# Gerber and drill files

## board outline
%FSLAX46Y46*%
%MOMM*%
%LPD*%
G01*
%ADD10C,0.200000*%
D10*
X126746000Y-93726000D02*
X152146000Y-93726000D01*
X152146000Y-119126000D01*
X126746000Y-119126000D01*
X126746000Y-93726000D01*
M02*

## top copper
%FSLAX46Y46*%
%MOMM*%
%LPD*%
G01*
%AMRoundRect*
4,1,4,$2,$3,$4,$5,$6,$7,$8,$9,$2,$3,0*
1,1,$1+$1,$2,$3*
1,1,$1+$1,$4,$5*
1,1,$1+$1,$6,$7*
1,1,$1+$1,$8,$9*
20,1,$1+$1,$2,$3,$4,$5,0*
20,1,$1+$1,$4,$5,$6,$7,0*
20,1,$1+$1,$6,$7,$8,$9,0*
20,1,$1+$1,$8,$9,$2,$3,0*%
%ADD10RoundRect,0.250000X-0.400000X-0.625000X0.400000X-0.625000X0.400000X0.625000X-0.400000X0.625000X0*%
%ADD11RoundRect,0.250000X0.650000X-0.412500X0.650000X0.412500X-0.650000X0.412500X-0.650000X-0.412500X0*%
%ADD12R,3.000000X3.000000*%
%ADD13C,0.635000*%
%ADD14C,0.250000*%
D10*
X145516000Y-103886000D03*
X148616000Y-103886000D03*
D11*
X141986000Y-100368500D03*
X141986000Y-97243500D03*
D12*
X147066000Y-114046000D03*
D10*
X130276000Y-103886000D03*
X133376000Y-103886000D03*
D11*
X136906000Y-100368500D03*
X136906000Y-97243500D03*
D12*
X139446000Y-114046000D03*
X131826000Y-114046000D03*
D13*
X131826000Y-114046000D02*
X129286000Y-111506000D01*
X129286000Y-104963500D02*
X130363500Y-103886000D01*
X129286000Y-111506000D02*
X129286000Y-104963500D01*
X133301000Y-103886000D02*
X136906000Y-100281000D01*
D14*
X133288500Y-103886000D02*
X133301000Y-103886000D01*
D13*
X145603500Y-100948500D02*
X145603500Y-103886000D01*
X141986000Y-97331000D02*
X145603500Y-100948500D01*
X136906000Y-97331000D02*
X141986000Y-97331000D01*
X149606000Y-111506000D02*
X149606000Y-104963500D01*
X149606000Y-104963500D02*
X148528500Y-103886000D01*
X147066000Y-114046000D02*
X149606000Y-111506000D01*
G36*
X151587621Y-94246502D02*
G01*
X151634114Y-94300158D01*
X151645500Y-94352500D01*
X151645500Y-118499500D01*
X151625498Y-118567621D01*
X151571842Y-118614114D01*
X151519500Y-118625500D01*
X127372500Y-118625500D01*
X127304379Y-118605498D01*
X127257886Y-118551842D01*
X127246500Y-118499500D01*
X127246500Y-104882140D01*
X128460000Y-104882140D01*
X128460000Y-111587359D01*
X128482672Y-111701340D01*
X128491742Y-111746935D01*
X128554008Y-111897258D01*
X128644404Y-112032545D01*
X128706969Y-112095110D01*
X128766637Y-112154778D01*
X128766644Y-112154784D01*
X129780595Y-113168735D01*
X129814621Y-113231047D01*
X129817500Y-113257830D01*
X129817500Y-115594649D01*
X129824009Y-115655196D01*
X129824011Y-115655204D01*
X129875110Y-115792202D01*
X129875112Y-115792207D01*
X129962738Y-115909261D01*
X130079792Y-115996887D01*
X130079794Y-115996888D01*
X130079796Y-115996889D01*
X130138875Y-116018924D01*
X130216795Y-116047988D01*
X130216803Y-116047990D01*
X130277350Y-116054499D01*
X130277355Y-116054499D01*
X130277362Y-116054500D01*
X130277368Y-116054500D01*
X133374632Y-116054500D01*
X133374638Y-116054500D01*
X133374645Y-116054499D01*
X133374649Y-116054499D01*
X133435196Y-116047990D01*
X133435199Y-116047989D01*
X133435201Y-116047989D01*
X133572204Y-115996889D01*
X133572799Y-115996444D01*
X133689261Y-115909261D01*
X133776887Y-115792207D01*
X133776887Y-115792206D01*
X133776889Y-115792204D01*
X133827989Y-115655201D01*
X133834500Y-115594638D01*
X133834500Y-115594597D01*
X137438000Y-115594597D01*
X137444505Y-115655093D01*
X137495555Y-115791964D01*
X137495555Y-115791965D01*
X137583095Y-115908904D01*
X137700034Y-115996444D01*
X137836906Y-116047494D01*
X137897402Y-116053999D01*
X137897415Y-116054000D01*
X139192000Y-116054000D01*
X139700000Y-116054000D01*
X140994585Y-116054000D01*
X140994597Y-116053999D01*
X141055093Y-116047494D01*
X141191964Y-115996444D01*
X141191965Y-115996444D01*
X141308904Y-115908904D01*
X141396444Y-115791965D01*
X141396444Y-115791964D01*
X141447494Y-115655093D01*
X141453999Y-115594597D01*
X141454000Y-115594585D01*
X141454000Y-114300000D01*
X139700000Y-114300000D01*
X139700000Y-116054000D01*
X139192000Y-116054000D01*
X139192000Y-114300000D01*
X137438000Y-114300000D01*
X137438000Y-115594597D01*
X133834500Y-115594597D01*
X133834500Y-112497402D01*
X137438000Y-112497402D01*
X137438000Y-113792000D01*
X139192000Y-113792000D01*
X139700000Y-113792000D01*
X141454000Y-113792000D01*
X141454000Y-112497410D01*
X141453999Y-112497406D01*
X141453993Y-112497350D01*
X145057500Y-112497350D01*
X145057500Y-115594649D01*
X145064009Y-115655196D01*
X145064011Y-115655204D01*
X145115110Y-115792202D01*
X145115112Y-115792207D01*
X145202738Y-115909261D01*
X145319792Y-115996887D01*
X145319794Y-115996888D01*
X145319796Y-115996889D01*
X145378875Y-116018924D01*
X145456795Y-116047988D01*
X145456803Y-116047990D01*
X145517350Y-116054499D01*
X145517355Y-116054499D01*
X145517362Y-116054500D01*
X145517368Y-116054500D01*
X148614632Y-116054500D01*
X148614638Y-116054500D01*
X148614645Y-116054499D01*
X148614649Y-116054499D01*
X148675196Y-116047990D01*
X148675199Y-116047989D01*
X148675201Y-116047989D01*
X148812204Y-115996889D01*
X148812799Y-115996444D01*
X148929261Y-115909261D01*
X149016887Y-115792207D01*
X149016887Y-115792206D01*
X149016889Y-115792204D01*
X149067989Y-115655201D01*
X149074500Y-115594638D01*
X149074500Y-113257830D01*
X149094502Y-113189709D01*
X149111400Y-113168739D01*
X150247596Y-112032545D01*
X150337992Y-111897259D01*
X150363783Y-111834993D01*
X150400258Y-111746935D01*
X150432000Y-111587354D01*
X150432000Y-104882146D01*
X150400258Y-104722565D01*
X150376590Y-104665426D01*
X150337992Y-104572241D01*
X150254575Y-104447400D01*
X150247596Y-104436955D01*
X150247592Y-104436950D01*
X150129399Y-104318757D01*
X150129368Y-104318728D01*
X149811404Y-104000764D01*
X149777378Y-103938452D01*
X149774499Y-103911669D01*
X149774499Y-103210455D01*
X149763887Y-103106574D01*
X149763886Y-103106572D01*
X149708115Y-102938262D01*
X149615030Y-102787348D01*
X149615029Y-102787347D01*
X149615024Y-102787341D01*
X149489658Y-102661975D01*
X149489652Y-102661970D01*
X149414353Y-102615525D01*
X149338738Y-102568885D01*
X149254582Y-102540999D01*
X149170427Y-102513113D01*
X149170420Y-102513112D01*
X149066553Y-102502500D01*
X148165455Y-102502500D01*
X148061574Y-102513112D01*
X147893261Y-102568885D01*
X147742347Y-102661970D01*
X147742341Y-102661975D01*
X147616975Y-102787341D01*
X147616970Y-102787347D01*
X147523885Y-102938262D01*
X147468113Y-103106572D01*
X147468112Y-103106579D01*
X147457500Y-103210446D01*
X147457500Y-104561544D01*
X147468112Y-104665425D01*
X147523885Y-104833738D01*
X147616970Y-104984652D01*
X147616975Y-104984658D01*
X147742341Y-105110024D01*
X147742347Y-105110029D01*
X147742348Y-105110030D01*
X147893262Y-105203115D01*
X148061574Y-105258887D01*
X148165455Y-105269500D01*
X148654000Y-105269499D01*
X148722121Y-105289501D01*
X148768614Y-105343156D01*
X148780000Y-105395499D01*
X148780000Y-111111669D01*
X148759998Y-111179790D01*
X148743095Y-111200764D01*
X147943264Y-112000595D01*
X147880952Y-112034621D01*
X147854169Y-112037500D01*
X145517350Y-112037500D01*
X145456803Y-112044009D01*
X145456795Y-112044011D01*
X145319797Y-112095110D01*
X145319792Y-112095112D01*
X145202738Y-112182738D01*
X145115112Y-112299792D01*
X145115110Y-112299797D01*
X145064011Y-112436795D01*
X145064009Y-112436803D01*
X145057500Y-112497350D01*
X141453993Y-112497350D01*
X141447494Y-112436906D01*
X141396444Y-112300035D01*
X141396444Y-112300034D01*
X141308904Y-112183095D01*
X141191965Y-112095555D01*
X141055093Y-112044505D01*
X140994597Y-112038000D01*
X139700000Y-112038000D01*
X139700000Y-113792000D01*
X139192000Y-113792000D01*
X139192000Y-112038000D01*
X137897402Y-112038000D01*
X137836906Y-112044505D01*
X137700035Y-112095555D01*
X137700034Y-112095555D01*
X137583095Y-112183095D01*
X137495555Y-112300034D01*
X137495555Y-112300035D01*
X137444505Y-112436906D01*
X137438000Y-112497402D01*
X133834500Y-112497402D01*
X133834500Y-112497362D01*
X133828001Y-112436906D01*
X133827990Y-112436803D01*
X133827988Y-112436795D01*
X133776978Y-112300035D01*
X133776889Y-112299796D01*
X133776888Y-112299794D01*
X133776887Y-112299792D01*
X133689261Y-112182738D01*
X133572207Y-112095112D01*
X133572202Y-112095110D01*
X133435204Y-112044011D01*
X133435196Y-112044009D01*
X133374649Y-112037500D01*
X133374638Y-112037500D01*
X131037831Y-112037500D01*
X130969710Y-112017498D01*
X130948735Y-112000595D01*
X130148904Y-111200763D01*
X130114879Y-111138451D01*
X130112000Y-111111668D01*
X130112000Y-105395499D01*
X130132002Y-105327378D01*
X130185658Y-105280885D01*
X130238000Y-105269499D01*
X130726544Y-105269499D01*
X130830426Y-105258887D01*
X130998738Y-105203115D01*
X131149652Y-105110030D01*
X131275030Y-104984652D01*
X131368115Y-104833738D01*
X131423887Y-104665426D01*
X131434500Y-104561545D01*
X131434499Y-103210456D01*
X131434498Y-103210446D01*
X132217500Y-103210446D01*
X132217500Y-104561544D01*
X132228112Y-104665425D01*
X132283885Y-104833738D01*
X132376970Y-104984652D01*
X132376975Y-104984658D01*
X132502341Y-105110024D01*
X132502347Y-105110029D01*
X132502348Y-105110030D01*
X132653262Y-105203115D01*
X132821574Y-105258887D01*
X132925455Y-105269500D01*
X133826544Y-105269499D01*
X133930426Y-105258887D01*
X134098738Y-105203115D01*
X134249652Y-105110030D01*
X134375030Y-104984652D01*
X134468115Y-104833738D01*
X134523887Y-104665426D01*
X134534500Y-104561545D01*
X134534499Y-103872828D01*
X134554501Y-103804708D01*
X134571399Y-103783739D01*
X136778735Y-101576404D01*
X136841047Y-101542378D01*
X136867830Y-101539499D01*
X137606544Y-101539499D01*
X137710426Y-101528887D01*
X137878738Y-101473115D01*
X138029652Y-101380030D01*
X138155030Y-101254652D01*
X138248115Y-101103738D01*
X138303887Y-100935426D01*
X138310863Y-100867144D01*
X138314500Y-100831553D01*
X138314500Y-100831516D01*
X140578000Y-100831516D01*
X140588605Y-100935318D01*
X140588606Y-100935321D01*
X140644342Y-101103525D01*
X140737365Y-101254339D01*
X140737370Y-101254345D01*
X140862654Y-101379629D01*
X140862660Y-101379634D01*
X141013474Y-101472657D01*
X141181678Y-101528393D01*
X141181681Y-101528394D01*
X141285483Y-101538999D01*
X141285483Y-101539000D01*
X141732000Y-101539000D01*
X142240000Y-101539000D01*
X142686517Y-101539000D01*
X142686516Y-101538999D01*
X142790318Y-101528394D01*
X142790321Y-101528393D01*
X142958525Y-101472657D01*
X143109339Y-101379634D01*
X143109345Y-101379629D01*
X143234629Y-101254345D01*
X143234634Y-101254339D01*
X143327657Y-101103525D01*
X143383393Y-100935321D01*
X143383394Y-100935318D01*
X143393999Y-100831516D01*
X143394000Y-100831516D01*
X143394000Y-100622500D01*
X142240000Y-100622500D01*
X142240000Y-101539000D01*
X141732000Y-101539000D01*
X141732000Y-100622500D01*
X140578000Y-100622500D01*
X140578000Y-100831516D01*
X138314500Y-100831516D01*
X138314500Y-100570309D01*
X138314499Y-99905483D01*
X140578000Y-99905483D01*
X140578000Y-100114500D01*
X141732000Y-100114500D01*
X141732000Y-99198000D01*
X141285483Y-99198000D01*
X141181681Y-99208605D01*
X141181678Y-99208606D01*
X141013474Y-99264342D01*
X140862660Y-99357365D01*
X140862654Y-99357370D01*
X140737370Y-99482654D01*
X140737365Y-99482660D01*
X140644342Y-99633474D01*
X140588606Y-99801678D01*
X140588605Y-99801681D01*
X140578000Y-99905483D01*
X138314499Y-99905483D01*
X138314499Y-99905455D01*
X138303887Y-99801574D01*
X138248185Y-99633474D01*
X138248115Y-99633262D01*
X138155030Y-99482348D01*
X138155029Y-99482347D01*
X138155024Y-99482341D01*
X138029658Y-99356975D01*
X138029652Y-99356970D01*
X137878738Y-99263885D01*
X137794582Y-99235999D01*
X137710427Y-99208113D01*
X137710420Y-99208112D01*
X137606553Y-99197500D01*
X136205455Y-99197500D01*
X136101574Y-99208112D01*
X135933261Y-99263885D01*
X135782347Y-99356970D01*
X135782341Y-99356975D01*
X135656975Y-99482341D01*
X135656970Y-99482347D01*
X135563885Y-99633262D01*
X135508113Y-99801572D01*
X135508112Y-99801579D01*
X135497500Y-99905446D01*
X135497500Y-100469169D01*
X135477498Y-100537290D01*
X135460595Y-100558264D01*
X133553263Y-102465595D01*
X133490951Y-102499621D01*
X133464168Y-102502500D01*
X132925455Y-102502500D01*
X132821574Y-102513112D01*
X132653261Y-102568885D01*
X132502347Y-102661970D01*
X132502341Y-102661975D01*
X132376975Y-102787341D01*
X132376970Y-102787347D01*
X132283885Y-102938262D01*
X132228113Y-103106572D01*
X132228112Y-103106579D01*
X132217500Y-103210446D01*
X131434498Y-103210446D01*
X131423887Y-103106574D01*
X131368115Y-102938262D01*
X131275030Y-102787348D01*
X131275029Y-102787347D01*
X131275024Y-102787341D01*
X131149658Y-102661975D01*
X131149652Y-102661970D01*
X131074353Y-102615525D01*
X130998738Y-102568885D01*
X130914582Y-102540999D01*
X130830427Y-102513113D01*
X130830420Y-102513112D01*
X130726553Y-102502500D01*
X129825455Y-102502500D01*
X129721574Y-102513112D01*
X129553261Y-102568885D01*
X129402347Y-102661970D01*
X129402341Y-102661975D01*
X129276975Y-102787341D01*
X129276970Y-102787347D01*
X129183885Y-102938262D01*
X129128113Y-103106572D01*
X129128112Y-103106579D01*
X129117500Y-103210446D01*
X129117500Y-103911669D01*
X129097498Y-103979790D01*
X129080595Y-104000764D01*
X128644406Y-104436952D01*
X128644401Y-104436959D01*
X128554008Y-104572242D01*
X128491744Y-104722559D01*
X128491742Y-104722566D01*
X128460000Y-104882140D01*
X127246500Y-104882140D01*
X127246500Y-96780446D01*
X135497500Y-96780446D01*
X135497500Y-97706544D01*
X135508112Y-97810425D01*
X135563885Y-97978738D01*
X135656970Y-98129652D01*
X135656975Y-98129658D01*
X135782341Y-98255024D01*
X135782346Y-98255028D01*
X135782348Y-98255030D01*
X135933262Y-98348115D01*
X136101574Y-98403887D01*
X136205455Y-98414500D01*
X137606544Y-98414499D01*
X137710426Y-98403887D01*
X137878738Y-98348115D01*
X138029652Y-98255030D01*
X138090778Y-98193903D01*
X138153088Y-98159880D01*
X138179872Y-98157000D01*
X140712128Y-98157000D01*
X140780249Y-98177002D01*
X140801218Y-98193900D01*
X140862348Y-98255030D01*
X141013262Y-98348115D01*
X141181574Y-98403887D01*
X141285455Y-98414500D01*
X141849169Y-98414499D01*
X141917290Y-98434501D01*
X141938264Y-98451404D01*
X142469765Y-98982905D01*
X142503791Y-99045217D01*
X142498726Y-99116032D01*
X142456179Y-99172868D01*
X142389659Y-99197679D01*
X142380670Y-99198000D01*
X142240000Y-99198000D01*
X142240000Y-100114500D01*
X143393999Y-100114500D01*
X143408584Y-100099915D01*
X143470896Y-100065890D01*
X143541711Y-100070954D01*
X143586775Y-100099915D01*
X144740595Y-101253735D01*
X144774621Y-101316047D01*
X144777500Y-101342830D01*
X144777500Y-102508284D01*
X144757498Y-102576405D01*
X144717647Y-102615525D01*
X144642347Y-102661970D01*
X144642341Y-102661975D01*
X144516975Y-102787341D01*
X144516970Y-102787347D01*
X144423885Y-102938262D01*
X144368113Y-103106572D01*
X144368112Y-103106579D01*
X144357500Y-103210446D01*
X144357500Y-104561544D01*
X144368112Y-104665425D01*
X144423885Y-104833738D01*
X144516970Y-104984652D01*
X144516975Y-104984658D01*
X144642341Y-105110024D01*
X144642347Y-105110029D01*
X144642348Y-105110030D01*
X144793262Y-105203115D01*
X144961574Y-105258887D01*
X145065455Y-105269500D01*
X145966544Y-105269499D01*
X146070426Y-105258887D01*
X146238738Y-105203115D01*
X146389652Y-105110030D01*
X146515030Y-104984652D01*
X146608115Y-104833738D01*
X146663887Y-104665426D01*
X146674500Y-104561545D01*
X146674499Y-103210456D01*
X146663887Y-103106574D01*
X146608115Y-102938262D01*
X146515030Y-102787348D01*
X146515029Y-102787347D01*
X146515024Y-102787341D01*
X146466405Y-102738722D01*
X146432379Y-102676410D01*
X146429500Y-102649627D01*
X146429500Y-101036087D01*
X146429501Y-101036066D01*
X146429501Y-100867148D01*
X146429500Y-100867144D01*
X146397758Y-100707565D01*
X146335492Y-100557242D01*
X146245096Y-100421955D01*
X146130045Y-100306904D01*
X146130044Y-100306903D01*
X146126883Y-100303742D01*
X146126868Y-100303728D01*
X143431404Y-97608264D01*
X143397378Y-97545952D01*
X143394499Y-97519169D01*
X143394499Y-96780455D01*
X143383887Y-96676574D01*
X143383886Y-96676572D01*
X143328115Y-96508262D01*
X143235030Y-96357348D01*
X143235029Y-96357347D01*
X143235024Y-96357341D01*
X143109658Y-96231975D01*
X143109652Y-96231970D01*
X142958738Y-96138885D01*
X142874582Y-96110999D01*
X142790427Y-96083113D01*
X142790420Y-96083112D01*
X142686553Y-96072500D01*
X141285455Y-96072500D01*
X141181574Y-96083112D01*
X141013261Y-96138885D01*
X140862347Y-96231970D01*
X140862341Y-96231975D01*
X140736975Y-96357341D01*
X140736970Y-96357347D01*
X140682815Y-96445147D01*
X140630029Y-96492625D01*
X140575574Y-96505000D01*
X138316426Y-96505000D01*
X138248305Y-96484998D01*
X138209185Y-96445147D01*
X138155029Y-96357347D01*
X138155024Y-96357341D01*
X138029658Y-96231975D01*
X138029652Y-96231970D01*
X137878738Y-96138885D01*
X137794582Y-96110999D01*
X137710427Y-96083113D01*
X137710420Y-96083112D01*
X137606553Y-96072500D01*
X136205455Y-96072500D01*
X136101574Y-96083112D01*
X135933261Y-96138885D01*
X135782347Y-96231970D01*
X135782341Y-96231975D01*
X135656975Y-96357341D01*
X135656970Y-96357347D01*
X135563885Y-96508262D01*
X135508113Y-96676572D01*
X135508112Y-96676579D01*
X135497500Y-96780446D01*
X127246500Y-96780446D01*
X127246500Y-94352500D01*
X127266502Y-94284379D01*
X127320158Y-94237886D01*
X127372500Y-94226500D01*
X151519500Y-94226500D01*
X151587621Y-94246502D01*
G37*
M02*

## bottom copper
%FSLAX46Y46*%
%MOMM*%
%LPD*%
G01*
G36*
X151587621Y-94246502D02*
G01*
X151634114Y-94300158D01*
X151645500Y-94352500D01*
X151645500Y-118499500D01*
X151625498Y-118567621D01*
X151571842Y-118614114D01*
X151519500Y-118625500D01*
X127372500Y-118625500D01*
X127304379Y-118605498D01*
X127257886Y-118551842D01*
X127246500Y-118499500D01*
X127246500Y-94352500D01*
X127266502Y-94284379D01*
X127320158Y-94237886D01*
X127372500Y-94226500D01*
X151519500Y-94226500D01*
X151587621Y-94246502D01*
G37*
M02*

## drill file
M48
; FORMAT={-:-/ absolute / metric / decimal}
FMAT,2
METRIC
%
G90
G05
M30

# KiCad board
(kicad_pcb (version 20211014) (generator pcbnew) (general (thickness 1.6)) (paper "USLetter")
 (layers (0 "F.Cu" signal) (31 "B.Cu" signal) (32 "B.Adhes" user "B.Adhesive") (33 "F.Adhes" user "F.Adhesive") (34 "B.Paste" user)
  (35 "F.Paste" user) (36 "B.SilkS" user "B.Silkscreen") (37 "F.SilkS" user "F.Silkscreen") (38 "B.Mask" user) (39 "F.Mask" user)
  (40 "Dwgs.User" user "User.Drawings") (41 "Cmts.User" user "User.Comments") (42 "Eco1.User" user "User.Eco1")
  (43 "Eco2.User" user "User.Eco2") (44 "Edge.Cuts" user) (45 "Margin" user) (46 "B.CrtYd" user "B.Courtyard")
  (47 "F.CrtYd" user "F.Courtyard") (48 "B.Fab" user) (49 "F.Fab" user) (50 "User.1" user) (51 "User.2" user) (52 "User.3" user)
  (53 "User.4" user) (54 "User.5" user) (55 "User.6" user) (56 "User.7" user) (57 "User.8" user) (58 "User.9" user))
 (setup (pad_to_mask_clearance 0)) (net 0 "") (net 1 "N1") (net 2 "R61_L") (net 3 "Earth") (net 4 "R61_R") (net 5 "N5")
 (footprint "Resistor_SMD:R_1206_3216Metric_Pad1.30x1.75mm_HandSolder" (layer "F.Cu") (at 147.066 103.886)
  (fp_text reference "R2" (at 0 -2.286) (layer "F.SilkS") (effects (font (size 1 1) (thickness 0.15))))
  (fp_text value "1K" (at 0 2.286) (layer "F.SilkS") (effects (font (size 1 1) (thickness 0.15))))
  (pad "1" smd roundrect (at -1.55 0) (size 1.3 1.75) (layers "F.Cu" "F.Paste" "F.Mask") (roundrect_rratio 0.1923076923) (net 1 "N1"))
  (pad "2" smd roundrect (at 1.55 0) (size 1.3 1.75) (layers "F.Cu" "F.Paste" "F.Mask") (roundrect_rratio 0.1923076923) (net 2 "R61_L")))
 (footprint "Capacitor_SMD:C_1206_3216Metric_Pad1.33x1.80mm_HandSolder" (layer "F.Cu") (at 141.986 98.806 90)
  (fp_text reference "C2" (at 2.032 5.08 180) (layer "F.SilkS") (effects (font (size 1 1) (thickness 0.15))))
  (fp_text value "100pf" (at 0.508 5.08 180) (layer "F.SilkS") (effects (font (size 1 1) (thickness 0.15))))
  (pad "1" smd roundrect (at -1.5625 0 90) (size 1.325 1.8) (layers "F.Cu" "F.Paste" "F.Mask") (roundrect_rratio 0.1886792453)
   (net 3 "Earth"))
  (pad "2" smd roundrect (at 1.5625 0 90) (size 1.325 1.8) (layers "F.Cu" "F.Paste" "F.Mask") (roundrect_rratio 0.1886792453) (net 1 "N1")))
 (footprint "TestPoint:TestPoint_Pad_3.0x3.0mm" (layer "F.Cu") (at 147.066 114.046)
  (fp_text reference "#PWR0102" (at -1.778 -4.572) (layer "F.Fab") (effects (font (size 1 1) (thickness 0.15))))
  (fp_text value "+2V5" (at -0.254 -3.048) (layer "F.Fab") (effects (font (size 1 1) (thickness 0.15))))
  (pad "1" smd rect (at 0 0) (size 3 3) (layers "F.Cu" "F.Paste" "F.Mask") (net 2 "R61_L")))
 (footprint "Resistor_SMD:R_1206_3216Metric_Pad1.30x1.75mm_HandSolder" (layer "F.Cu") (at 131.826 103.886)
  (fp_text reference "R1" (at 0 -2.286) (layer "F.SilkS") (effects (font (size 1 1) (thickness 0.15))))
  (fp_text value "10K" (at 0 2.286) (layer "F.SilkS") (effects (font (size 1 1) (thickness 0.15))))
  (pad "1" smd roundrect (at -1.55 0) (size 1.3 1.75) (layers "F.Cu" "F.Paste" "F.Mask") (roundrect_rratio 0.1923076923) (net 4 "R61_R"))
  (pad "2" smd roundrect (at 1.55 0) (size 1.3 1.75) (layers "F.Cu" "F.Paste" "F.Mask") (roundrect_rratio 0.1923076923) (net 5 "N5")))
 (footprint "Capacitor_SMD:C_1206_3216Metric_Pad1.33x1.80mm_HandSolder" (layer "F.Cu") (at 136.906 98.806 90)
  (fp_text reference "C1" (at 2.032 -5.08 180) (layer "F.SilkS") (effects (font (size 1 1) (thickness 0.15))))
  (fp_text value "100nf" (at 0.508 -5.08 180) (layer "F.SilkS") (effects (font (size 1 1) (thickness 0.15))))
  (pad "1" smd roundrect (at -1.5625 0 90) (size 1.325 1.8) (layers "F.Cu" "F.Paste" "F.Mask") (roundrect_rratio 0.1886792453) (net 5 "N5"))
  (pad "2" smd roundrect (at 1.5625 0 90) (size 1.325 1.8) (layers "F.Cu" "F.Paste" "F.Mask") (roundrect_rratio 0.1886792453) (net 1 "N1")))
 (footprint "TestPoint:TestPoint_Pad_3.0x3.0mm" (layer "F.Cu") (at 139.446 114.046)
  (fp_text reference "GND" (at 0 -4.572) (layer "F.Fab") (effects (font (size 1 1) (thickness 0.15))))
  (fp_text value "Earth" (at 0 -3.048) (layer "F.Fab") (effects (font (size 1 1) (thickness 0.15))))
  (pad "1" smd rect (at 0 0) (size 3 3) (layers "F.Cu" "F.Paste" "F.Mask") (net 3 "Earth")))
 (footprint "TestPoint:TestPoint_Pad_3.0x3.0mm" (layer "F.Cu") (at 131.826 114.046)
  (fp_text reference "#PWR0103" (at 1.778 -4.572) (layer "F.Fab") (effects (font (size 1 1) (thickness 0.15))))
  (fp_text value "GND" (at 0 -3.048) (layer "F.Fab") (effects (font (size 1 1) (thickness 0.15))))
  (pad "1" smd rect (at 0 0) (size 3 3) (layers "F.Cu" "F.Paste" "F.Mask") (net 4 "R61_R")))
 (gr_rect (start 126.746 93.726) (end 152.146 119.126) (layer "Edge.Cuts") (width 0.2) (fill none))
 (segment (start 131.826 114.046) (end 129.286 111.506) (width 0.635) (layer "F.Cu") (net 4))
 (segment (start 129.286 104.9635) (end 130.3635 103.886) (width 0.635) (layer "F.Cu") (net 4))
 (segment (start 129.286 111.506) (end 129.286 104.9635) (width 0.635) (layer "F.Cu") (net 4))
 (segment (start 133.301 103.886) (end 136.906 100.281) (width 0.635) (layer "F.Cu") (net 5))
 (segment (start 133.2885 103.886) (end 133.301 103.886) (width 0.25) (layer "F.Cu") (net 5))
 (segment (start 145.6035 100.9485) (end 145.6035 103.886) (width 0.635) (layer "F.Cu") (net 1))
 (segment (start 141.986 97.331) (end 145.6035 100.9485) (width 0.635) (layer "F.Cu") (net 1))
 (segment (start 136.906 97.331) (end 141.986 97.331) (width 0.635) (layer "F.Cu") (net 1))
 (segment (start 149.606 111.506) (end 149.606 104.9635) (width 0.635) (layer "F.Cu") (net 2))
 (segment (start 149.606 104.9635) (end 148.5285 103.886) (width 0.635) (layer "F.Cu") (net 2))
 (segment (start 147.066 114.046) (end 149.606 111.506) (width 0.635) (layer "F.Cu") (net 2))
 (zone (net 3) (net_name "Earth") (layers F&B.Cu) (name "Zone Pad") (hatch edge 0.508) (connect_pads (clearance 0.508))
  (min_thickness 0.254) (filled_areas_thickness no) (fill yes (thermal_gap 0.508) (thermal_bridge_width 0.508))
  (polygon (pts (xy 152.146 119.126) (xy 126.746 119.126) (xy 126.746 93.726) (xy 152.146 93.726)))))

